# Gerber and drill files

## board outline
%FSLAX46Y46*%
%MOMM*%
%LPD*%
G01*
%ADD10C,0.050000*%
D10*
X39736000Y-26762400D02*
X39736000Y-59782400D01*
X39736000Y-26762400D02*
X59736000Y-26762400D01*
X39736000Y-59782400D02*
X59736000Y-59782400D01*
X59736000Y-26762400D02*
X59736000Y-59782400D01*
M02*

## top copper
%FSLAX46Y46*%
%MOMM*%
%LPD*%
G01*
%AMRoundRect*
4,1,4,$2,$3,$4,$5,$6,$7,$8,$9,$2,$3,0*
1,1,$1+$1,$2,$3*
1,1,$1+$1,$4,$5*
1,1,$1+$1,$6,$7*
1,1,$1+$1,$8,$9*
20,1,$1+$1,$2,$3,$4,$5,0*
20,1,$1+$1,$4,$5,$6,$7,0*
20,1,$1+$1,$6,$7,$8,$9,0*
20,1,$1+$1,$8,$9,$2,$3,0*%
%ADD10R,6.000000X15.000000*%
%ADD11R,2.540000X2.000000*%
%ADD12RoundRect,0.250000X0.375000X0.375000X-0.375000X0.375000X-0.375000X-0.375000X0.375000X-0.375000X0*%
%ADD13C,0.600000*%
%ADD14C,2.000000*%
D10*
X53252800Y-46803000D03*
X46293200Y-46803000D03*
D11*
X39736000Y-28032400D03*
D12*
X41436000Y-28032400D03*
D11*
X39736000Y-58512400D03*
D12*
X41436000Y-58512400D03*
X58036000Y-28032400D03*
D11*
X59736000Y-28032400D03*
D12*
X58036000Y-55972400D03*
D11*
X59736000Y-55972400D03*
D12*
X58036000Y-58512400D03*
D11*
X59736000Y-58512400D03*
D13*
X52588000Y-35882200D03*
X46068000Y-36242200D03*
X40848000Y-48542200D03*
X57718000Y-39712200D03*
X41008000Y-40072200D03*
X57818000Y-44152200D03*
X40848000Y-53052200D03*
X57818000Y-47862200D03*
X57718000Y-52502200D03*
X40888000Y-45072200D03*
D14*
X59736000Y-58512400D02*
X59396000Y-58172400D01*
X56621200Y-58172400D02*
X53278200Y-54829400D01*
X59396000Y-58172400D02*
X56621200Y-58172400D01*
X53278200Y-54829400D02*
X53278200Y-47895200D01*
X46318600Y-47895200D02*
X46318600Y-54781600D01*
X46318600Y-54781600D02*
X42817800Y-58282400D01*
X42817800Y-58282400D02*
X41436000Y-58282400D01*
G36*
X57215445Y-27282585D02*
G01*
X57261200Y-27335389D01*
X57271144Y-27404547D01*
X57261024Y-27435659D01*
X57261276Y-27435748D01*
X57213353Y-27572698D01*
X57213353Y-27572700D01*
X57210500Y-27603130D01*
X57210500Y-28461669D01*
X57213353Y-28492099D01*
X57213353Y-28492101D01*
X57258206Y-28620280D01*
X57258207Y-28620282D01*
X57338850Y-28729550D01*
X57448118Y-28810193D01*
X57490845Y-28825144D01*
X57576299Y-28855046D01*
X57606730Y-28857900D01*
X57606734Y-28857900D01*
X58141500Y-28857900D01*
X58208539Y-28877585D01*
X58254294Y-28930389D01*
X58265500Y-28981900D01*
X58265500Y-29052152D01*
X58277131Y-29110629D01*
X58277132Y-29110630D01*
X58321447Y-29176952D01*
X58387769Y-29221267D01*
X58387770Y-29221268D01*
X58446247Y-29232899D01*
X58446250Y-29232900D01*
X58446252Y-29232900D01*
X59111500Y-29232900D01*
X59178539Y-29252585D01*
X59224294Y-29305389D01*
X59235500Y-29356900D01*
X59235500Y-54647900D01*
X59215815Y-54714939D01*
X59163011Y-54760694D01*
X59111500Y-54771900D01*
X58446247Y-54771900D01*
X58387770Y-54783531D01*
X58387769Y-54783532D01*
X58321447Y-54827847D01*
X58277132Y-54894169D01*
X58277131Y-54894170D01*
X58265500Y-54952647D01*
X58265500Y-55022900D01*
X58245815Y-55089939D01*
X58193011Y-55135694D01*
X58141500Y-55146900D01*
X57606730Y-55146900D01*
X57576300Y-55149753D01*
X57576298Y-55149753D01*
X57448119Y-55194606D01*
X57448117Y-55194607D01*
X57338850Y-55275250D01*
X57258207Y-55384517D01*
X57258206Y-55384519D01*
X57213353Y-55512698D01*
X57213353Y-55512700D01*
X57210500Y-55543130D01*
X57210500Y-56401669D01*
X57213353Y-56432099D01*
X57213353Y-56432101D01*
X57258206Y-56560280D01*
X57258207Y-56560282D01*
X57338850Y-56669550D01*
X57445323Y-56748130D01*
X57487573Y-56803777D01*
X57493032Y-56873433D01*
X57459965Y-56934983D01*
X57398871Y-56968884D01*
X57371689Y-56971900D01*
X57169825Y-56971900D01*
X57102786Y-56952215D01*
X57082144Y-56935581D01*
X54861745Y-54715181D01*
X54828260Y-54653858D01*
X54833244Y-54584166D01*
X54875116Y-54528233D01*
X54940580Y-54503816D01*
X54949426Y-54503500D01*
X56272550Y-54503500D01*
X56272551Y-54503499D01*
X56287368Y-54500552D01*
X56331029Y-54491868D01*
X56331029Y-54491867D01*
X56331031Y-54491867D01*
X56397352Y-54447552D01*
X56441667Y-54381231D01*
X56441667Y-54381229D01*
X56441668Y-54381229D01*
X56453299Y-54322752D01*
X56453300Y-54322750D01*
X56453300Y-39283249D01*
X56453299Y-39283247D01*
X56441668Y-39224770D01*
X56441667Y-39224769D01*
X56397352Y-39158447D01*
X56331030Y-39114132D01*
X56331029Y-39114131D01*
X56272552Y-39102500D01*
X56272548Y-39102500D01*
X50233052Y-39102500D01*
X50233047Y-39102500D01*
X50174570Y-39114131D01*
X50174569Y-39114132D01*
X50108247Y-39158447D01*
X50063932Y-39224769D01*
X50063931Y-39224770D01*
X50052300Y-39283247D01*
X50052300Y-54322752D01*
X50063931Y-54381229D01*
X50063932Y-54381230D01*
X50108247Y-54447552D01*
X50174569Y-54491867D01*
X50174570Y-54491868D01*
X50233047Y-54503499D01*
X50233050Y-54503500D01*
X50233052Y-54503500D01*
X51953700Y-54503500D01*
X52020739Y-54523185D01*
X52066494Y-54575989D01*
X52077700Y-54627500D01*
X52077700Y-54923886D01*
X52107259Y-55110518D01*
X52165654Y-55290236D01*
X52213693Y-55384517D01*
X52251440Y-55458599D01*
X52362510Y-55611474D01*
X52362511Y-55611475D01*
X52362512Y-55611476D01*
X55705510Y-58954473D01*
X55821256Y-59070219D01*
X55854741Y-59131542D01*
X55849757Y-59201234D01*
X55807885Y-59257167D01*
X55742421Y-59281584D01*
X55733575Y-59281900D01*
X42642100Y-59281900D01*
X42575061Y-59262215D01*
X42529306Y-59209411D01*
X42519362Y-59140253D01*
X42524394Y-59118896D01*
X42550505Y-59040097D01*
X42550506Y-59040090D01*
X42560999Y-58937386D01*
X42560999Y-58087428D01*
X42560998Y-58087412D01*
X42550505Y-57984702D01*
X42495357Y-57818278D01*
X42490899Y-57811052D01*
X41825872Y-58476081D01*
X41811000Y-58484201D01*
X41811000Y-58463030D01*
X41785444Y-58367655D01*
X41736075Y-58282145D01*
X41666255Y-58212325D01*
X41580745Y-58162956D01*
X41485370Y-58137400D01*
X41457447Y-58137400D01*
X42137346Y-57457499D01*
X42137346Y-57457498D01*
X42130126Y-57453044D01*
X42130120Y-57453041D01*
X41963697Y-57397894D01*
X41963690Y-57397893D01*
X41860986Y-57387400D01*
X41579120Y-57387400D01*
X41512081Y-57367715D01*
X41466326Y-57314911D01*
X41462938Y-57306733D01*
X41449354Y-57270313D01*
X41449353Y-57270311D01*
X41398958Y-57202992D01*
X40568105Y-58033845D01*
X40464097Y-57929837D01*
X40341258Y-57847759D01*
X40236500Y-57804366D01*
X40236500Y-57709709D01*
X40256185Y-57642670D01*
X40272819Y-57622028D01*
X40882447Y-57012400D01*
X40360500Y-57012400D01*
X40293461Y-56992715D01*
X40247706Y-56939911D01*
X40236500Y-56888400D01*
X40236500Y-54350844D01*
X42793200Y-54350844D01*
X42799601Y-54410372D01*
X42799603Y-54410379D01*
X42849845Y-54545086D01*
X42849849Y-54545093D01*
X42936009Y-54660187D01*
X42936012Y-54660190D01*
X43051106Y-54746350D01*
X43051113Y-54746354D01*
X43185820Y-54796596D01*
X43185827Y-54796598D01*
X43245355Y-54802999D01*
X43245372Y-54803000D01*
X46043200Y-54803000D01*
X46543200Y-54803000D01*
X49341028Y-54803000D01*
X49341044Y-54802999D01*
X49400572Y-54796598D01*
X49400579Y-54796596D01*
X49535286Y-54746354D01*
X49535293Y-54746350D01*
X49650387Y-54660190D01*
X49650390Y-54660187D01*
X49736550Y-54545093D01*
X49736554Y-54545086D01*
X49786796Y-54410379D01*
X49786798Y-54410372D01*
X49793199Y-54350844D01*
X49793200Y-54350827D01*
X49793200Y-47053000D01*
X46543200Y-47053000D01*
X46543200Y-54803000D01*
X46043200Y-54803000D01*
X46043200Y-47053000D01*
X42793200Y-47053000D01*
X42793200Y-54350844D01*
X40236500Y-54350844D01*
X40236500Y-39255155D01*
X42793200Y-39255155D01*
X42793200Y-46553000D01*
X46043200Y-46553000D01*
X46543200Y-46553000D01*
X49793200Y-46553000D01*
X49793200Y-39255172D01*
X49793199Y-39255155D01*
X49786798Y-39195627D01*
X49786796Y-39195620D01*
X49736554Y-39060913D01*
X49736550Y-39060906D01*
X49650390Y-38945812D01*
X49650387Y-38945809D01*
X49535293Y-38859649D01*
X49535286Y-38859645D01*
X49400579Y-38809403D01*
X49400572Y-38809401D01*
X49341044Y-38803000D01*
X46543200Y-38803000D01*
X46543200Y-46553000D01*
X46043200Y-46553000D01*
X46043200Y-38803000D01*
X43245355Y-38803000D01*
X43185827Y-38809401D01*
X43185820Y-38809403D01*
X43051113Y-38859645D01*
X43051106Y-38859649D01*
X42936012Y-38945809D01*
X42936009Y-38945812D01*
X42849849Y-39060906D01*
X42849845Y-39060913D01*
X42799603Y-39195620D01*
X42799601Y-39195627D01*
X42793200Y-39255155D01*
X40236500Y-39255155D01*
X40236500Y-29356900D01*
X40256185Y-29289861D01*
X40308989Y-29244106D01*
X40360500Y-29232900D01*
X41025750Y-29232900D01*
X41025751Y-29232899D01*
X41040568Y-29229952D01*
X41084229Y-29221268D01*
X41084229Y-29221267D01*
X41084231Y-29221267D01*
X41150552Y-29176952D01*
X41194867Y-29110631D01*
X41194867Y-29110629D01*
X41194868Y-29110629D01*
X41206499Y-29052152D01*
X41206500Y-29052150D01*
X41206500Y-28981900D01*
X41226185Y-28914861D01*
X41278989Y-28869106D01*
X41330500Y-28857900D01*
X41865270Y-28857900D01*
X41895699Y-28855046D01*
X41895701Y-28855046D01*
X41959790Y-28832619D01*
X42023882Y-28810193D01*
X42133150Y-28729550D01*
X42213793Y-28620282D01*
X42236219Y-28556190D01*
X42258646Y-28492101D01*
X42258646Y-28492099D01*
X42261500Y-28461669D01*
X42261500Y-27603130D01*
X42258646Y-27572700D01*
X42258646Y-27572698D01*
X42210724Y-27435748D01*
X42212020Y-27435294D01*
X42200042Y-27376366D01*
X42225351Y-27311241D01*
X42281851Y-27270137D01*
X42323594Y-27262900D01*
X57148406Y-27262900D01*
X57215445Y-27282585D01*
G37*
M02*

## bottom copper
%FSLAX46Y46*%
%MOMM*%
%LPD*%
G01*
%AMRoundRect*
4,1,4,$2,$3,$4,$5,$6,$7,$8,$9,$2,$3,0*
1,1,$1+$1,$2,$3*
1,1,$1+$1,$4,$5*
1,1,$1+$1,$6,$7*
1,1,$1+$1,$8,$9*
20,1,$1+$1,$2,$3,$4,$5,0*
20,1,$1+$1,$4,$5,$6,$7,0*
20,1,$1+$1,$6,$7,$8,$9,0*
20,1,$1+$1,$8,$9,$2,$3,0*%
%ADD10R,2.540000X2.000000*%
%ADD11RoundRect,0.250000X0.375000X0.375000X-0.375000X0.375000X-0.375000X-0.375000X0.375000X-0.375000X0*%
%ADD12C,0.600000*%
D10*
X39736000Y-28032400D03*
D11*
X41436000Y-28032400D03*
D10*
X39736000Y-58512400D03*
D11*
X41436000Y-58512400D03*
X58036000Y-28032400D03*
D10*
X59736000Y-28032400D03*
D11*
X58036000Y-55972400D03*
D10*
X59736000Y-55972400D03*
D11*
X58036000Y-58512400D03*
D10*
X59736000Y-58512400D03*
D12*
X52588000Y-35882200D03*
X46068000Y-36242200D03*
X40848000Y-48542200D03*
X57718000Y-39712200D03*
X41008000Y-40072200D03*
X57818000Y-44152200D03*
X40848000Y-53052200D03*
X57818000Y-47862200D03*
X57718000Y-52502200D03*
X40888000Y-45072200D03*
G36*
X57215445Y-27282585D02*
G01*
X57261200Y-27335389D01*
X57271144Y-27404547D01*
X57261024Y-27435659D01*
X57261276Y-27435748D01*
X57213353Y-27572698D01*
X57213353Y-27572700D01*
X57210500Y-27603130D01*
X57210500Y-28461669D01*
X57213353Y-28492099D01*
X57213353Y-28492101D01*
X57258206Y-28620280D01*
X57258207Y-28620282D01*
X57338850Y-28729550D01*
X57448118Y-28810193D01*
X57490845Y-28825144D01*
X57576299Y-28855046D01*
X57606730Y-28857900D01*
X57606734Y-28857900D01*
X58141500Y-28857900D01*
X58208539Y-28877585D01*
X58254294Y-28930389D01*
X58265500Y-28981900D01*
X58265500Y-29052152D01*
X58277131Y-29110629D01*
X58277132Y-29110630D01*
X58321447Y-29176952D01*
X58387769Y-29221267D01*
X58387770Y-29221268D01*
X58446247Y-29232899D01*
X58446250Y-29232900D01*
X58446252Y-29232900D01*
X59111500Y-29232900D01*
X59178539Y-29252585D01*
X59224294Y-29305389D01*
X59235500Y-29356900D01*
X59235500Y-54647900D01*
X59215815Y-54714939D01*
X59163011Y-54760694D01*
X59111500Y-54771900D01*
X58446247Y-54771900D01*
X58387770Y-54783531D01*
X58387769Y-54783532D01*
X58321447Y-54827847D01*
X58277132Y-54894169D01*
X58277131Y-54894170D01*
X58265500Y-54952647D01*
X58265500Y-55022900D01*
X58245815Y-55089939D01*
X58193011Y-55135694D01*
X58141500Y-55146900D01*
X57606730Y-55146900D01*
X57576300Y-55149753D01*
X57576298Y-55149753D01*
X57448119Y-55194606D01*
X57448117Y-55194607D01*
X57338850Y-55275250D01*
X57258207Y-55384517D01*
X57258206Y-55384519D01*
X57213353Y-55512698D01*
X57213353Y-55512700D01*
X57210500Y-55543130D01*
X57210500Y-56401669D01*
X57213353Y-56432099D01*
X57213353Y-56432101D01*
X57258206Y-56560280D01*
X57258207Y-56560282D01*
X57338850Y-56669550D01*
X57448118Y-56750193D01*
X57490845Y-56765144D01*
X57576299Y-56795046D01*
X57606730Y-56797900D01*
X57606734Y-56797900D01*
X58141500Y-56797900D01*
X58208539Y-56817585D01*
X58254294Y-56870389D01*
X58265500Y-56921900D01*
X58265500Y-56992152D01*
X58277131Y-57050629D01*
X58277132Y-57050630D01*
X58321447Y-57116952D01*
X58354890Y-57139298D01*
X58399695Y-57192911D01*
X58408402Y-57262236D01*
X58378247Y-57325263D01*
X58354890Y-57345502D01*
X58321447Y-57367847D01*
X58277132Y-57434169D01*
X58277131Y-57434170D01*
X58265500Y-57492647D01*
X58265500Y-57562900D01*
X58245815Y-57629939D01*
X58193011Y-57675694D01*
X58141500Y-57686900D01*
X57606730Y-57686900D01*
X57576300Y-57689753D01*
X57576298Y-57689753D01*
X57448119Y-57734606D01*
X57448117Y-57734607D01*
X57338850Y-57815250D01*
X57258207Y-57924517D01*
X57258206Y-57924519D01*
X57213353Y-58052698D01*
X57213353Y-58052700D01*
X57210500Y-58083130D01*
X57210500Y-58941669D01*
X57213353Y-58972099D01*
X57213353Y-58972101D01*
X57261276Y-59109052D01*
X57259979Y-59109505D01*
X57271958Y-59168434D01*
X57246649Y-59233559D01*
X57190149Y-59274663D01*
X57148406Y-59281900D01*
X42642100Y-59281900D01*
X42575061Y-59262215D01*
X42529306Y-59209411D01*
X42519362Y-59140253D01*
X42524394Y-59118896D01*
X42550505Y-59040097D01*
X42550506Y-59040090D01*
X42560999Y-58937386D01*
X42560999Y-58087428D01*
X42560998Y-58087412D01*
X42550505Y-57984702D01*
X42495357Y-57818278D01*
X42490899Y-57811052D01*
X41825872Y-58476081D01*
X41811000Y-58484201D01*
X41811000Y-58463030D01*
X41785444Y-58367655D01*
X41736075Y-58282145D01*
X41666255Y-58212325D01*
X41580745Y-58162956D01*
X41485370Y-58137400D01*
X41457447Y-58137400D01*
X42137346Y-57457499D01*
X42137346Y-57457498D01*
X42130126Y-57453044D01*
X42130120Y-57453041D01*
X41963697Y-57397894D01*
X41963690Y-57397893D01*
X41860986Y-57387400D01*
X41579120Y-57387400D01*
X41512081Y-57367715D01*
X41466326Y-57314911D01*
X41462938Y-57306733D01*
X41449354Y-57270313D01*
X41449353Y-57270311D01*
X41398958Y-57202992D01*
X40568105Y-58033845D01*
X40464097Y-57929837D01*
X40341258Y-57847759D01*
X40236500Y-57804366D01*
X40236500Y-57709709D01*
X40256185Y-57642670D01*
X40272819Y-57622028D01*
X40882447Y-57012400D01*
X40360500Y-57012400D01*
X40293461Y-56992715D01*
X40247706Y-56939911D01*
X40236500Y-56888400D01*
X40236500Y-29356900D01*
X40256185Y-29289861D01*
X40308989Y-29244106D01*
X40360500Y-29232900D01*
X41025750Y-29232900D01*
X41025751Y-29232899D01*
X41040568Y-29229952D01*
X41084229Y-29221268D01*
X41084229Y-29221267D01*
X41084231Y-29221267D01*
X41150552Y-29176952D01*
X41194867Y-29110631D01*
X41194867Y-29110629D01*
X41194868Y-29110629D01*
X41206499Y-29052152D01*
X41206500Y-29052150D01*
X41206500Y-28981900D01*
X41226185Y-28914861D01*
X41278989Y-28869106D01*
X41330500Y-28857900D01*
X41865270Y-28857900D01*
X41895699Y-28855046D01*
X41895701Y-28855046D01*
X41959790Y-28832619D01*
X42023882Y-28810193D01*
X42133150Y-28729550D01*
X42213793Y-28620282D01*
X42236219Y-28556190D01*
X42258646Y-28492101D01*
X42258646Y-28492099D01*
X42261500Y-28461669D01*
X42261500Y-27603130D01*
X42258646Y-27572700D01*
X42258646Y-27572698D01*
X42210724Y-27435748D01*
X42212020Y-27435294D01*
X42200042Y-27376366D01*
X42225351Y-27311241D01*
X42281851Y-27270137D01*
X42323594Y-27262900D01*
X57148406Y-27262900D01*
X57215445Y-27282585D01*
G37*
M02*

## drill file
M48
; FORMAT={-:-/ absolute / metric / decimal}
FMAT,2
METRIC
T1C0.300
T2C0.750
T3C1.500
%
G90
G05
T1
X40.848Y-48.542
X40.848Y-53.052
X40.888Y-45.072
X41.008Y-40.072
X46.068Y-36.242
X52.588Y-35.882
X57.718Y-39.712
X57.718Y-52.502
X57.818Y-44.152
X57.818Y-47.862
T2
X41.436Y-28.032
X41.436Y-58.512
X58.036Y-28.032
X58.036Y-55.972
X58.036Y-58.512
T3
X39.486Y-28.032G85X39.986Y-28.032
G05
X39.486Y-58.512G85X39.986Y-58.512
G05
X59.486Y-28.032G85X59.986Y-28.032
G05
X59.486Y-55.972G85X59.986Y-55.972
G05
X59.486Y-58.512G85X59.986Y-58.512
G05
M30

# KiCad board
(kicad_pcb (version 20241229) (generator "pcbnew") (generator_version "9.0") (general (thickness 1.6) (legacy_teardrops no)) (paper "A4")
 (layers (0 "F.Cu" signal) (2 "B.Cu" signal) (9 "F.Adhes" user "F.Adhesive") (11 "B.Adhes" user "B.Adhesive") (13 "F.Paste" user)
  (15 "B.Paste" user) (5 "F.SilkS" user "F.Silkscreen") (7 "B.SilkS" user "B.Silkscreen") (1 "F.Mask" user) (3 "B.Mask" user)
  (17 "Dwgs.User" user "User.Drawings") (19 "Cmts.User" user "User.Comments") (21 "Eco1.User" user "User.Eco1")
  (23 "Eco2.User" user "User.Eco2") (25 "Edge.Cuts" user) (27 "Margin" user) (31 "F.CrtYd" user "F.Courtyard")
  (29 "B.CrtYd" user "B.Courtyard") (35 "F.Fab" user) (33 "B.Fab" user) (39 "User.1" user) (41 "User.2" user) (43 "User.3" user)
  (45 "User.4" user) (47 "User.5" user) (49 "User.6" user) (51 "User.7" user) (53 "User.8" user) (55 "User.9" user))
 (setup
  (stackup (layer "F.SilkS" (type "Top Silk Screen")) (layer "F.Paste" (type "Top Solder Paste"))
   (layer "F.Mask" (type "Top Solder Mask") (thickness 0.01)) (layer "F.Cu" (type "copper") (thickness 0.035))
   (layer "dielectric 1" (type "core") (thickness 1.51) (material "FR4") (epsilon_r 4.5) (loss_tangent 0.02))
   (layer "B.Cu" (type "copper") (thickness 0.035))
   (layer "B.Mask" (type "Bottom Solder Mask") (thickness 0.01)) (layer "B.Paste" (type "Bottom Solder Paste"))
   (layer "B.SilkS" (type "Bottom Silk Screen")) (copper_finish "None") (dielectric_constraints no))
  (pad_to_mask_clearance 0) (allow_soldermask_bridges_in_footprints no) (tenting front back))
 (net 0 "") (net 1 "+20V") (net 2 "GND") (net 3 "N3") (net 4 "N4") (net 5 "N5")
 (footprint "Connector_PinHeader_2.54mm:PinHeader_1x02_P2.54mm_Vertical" (layer "F.Cu") (at 50.789 40.5546 -90)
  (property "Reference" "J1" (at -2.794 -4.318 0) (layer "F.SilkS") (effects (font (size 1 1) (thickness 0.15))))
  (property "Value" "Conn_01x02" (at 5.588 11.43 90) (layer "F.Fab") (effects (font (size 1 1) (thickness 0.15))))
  (pad "1" smd rect (at 6.2484 -2.4638) (size 6 15) (layers "F.Cu" "F.Mask" "F.Paste") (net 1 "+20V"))
  (pad "2" smd rect (at 6.2484 4.4958) (size 6 15) (layers "F.Cu" "F.Mask" "F.Paste") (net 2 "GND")))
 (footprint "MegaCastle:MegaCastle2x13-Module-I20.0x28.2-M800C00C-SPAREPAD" (layer "F.Cu") (at 49.736 43.2724)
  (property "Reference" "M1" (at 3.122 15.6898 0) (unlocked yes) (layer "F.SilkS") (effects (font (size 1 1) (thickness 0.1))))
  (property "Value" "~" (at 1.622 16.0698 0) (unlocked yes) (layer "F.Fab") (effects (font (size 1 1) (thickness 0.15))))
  (fp_line (start -10 -16.51) (end -10 16.51) (stroke (width 0.05) (type default)) (layer "Edge.Cuts"))
  (fp_line (start -10 -16.51) (end 10 -16.51) (stroke (width 0.05) (type default)) (layer "Edge.Cuts"))
  (fp_line (start -10 16.51) (end 10 16.51) (stroke (width 0.05) (type default)) (layer "Edge.Cuts"))
  (fp_line (start 10 -16.51) (end 10 16.51) (stroke (width 0.05) (type default)) (layer "Edge.Cuts"))
  (pad "1" thru_hole rect (at -10 -15.24) (size 2.54 2) (drill oval 2 1.5) (layers "*.Cu" "*.Mask") (remove_unused_layers no) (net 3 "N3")
   (thermal_bridge_angle 45))
  (pad "1" thru_hole roundrect (at -8.3 -15.24 180) (size 1.25 1.25) (drill 0.75) (layers "*.Cu" "*.Mask") (remove_unused_layers no)
   (roundrect_rratio 0.2) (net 3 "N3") (thermal_bridge_angle 45))
  (pad "13" thru_hole rect (at -10 15.24) (size 2.54 2) (drill oval 2 1.5) (layers "*.Cu" "*.Mask") (remove_unused_layers no) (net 2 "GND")
   (thermal_bridge_angle 45))
  (pad "13" thru_hole roundrect (at -8.3 15.24 180) (size 1.25 1.25) (drill 0.75) (layers "*.Cu" "*.Mask") (remove_unused_layers no)
   (roundrect_rratio 0.2) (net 2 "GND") (thermal_bridge_angle 45))
  (pad "14" thru_hole roundrect (at 8.3 -15.24 180) (size 1.25 1.25) (drill 0.75) (layers "*.Cu" "*.Mask") (remove_unused_layers no)
   (roundrect_rratio 0.2) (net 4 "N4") (thermal_bridge_angle 45))
  (pad "14" thru_hole rect (at 10 -15.24) (size 2.54 2) (drill oval 2 1.5) (layers "*.Cu" "*.Mask") (remove_unused_layers no) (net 4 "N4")
   (thermal_bridge_angle 45))
  (pad "25" thru_hole roundrect (at 8.3 12.7 180) (size 1.25 1.25) (drill 0.75) (layers "*.Cu" "*.Mask") (remove_unused_layers no)
   (roundrect_rratio 0.2) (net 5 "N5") (thermal_bridge_angle 45))
  (pad "25" thru_hole rect (at 10 12.7) (size 2.54 2) (drill oval 2 1.5) (layers "*.Cu" "*.Mask") (remove_unused_layers no) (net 5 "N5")
   (thermal_bridge_angle 45))
  (pad "26" thru_hole roundrect (at 8.3 15.24 180) (size 1.25 1.25) (drill 0.75) (layers "*.Cu" "*.Mask") (remove_unused_layers no)
   (roundrect_rratio 0.2) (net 1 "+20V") (thermal_bridge_angle 45))
  (pad "26" thru_hole rect (at 10 15.24) (size 2.54 2) (drill oval 2 1.5) (layers "*.Cu" "*.Mask") (remove_unused_layers no) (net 1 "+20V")
   (thermal_bridge_angle 45))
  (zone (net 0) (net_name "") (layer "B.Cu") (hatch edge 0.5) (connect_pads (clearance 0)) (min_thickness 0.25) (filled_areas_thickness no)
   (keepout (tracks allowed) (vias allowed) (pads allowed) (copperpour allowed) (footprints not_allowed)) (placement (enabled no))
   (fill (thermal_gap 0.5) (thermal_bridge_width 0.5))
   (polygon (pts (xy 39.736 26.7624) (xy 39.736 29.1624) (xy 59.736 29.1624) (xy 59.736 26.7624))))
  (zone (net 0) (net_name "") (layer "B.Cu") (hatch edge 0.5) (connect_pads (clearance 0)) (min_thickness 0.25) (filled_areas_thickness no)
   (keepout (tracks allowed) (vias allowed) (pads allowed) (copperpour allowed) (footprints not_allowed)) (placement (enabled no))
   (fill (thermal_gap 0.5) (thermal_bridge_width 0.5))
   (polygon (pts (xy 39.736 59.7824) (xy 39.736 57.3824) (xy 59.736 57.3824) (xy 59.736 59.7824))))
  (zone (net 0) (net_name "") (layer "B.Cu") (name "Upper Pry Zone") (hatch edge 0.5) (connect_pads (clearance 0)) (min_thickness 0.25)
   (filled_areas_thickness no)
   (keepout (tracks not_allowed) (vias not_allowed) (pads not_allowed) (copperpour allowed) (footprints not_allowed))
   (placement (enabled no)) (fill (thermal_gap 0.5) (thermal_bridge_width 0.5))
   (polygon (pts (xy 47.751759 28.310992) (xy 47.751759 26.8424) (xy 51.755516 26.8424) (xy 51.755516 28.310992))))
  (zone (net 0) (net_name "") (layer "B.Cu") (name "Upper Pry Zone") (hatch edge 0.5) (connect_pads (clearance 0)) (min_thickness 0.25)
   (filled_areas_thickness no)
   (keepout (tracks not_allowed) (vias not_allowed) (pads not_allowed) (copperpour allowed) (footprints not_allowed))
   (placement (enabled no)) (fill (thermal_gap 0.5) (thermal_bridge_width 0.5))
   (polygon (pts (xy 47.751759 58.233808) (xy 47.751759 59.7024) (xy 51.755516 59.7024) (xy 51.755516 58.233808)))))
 (segment (start 59.736 58.5124) (end 59.396 58.1724) (width 2) (layer "F.Cu") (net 1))
 (segment (start 56.6212 58.1724) (end 53.2782 54.8294) (width 2) (layer "F.Cu") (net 1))
 (segment (start 59.396 58.1724) (end 56.6212 58.1724) (width 2) (layer "F.Cu") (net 1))
 (segment (start 53.2782 54.8294) (end 53.2782 47.8952) (width 2) (layer "F.Cu") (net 1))
 (segment (start 46.3186 47.8952) (end 46.3186 54.7816) (width 2) (layer "F.Cu") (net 2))
 (segment (start 46.3186 54.7816) (end 42.8178 58.2824) (width 2) (layer "F.Cu") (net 2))
 (segment (start 42.8178 58.2824) (end 41.436 58.2824) (width 2) (layer "F.Cu") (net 2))
 (via (at 52.588 35.8822) (size 0.6) (drill 0.3) (layers "F.Cu" "B.Cu") (free yes) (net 2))
 (via (at 46.068 36.2422) (size 0.6) (drill 0.3) (layers "F.Cu" "B.Cu") (free yes) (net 2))
 (via (at 40.848 48.5422) (size 0.6) (drill 0.3) (layers "F.Cu" "B.Cu") (free yes) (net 2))
 (via (at 57.718 39.7122) (size 0.6) (drill 0.3) (layers "F.Cu" "B.Cu") (free yes) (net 2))
 (via (at 41.008 40.0722) (size 0.6) (drill 0.3) (layers "F.Cu" "B.Cu") (free yes) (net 2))
 (via (at 57.818 44.1522) (size 0.6) (drill 0.3) (layers "F.Cu" "B.Cu") (free yes) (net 2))
 (via (at 40.848 53.0522) (size 0.6) (drill 0.3) (layers "F.Cu" "B.Cu") (free yes) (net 2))
 (via (at 57.818 47.8622) (size 0.6) (drill 0.3) (layers "F.Cu" "B.Cu") (free yes) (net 2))
 (via (at 57.718 52.5022) (size 0.6) (drill 0.3) (layers "F.Cu" "B.Cu") (free yes) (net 2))
 (via (at 40.888 45.0722) (size 0.6) (drill 0.3) (layers "F.Cu" "B.Cu") (free yes) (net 2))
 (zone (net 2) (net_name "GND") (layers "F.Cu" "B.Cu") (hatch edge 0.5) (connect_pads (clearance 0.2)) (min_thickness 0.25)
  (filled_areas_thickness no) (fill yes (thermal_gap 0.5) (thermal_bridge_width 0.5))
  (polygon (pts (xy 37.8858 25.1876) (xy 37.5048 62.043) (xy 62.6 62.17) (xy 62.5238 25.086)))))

